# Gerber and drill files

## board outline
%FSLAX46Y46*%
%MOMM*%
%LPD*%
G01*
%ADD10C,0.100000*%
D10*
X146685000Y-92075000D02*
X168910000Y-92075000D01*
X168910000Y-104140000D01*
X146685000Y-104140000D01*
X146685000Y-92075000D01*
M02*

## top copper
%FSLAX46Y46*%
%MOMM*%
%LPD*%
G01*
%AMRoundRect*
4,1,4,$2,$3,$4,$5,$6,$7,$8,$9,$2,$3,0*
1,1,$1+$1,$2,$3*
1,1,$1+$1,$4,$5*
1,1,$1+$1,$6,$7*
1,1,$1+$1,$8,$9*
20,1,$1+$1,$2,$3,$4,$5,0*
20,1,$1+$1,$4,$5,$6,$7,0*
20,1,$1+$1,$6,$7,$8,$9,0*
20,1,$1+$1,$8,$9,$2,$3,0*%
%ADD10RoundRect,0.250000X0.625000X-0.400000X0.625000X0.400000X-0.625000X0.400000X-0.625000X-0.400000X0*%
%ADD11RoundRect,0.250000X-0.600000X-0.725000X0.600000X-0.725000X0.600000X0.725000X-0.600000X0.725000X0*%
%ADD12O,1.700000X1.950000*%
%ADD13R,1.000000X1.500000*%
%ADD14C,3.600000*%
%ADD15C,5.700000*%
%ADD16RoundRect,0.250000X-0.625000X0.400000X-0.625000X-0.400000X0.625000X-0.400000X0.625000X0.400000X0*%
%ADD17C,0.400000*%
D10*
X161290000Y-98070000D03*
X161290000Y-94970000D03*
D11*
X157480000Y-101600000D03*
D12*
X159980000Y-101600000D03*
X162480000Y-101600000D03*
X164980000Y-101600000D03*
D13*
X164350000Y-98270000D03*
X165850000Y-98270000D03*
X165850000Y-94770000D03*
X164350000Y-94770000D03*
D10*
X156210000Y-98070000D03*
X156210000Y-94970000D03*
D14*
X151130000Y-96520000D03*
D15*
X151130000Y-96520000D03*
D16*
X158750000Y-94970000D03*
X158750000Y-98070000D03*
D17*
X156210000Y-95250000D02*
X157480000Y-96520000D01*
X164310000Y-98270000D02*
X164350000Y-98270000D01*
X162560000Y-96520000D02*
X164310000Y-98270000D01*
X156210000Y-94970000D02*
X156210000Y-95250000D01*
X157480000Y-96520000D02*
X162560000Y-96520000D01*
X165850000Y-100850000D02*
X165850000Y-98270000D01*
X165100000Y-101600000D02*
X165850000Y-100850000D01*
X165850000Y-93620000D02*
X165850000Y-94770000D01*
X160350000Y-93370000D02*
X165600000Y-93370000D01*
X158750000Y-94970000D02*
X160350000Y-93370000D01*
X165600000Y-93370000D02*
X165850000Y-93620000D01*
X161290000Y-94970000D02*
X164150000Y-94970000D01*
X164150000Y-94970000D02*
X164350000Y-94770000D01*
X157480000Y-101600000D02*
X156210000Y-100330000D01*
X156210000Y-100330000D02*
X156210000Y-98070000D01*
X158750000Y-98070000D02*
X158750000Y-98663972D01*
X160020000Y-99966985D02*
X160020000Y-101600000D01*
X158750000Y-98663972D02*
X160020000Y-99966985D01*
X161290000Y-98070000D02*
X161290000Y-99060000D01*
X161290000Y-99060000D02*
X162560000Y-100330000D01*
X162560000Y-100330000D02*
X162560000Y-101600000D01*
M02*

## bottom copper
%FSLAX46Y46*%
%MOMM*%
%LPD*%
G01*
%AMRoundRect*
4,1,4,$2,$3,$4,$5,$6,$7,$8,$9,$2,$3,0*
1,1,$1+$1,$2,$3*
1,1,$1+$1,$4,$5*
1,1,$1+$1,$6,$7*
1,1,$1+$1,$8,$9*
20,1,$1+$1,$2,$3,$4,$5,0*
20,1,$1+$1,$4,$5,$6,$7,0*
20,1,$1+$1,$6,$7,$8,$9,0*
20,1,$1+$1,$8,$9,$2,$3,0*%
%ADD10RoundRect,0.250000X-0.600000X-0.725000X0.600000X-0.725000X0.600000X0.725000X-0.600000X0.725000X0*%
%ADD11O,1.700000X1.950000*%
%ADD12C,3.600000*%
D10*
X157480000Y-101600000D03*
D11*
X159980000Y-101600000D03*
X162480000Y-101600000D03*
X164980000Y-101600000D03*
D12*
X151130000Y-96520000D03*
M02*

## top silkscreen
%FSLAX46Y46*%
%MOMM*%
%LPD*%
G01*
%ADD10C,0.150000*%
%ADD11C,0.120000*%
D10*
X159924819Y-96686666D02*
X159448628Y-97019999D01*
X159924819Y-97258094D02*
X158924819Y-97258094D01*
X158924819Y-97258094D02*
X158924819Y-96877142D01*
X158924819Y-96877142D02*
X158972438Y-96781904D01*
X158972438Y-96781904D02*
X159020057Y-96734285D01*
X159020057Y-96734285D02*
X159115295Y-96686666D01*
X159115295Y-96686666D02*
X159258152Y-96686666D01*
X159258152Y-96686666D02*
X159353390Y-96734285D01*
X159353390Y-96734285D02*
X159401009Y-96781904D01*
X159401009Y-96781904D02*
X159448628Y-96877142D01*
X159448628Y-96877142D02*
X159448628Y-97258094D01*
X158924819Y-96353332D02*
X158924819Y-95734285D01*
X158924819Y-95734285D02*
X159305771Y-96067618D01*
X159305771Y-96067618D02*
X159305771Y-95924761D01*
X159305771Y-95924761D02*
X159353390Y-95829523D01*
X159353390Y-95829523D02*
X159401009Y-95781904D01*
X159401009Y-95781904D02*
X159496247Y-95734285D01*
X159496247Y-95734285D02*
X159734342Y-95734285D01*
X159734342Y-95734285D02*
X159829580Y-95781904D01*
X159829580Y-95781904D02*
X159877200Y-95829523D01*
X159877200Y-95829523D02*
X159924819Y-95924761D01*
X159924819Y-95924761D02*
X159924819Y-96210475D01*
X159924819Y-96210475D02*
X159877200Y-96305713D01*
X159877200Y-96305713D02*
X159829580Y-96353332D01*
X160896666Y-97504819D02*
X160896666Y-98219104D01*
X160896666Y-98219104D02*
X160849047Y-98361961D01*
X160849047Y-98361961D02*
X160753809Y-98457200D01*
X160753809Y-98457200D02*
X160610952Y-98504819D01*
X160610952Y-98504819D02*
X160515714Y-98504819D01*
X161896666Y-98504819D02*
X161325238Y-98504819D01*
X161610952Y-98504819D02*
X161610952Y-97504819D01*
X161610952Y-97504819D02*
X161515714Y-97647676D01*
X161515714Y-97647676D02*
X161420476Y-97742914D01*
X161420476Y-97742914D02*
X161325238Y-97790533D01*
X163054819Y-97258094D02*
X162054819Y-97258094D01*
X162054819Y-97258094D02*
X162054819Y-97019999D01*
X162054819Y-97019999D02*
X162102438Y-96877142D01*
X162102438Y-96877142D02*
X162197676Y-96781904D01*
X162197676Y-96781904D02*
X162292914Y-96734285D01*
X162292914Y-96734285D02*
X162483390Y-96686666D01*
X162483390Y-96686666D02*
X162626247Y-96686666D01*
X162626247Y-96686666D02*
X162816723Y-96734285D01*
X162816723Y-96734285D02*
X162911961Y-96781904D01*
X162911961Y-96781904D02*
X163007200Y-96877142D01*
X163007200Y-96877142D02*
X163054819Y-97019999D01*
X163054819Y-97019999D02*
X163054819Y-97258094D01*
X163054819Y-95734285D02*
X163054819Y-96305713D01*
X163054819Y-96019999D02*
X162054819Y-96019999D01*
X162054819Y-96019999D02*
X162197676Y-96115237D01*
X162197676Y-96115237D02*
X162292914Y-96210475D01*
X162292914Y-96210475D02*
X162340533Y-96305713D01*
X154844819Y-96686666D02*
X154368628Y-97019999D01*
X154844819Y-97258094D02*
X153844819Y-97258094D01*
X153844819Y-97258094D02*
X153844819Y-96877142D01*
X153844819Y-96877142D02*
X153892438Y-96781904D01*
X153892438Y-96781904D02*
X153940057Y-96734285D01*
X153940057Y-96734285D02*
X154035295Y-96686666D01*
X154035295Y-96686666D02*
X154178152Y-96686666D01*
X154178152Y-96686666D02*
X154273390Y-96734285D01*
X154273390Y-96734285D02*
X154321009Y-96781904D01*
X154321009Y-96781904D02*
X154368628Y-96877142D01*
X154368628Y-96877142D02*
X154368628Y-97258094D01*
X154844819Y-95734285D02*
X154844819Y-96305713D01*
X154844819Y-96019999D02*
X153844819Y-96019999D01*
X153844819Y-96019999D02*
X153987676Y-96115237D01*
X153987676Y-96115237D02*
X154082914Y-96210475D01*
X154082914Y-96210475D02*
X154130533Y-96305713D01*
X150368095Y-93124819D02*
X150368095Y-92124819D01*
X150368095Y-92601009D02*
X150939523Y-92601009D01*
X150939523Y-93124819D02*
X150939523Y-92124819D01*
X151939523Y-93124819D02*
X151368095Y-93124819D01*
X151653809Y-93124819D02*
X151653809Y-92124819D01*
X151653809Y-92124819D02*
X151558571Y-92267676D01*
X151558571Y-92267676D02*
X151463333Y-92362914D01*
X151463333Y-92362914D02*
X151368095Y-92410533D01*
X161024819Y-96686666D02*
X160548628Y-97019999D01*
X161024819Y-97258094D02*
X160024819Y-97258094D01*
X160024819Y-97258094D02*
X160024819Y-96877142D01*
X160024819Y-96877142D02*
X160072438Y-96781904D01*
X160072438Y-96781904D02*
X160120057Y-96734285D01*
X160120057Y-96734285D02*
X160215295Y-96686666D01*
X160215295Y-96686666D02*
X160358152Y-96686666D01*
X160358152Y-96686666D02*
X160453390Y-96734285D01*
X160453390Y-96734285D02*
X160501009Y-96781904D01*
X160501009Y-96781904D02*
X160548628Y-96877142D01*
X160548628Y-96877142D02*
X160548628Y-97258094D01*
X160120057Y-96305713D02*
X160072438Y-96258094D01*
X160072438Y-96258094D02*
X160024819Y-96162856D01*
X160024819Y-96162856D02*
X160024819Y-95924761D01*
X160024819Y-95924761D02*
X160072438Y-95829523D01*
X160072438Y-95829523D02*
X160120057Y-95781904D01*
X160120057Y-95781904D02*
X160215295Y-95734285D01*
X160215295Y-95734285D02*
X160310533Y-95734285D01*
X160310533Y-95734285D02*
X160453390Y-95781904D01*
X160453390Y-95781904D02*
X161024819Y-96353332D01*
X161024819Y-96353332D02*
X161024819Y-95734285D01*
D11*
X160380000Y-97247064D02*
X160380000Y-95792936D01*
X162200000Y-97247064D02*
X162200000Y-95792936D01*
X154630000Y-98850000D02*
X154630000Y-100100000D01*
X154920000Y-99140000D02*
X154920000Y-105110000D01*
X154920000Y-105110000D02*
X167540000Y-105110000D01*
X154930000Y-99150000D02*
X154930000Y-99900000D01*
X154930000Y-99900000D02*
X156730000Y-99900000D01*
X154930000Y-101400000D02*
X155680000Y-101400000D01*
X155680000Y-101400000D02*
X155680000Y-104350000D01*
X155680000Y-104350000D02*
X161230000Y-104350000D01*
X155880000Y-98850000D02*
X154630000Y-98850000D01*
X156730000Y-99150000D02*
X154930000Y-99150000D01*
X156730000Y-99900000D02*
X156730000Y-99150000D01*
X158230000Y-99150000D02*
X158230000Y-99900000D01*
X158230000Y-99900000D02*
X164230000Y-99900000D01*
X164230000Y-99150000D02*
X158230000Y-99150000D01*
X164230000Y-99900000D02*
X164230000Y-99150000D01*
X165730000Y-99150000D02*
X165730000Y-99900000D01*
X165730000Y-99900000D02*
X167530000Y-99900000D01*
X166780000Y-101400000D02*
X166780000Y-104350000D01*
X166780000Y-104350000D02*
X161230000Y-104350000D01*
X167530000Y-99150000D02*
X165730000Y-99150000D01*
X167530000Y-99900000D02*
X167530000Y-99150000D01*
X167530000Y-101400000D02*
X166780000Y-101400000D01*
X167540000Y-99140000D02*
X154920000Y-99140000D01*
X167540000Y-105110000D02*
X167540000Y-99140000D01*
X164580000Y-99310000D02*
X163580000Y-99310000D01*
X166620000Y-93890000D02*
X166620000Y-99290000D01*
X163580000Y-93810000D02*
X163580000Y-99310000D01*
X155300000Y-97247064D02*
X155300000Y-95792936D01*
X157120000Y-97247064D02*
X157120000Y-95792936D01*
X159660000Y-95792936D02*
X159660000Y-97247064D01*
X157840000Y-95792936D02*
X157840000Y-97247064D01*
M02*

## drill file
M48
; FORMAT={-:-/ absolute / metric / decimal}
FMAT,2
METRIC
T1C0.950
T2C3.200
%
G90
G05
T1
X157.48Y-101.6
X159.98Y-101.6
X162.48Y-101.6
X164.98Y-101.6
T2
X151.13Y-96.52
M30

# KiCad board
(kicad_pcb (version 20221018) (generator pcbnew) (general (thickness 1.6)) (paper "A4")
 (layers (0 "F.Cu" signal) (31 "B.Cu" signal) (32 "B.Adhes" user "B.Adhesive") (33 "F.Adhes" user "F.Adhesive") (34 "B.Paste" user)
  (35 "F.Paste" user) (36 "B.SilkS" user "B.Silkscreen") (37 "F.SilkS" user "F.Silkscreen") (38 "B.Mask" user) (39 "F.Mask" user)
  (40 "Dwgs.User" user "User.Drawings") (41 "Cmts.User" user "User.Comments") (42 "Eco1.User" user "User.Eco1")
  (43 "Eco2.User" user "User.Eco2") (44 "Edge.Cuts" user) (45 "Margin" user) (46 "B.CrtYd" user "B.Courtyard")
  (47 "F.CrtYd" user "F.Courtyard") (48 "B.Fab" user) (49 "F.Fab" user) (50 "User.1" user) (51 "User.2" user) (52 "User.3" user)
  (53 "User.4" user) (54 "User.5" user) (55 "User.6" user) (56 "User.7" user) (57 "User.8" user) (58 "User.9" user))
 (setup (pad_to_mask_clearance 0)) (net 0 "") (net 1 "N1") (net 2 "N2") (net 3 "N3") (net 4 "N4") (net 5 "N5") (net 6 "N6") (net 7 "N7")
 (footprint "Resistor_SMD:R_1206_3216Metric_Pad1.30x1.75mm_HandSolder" (layer "F.Cu") (at 161.29 96.52 90)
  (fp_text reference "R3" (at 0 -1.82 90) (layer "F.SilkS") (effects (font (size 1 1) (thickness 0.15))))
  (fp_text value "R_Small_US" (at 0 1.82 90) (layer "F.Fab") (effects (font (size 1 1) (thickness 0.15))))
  (fp_line (start -0.727064 -0.91) (end 0.727064 -0.91) (stroke (width 0.12) (type solid)) (layer "F.SilkS"))
  (fp_line (start -0.727064 0.91) (end 0.727064 0.91) (stroke (width 0.12) (type solid)) (layer "F.SilkS"))
  (pad "1" smd roundrect (at -1.55 0 90) (size 1.3 1.75) (layers "F.Cu" "F.Paste" "F.Mask") (roundrect_rratio 0.1923076923) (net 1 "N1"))
  (pad "2" smd roundrect (at 1.55 0 90) (size 1.3 1.75) (layers "F.Cu" "F.Paste" "F.Mask") (roundrect_rratio 0.1923076923) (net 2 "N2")))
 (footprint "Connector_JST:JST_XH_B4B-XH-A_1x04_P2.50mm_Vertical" (layer "F.Cu") (at 157.48 101.6)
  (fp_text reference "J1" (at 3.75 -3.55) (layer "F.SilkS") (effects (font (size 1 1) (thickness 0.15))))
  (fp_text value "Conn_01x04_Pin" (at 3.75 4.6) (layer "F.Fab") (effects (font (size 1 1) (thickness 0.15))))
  (fp_line (start -2.85 -2.75) (end -2.85 -1.5) (stroke (width 0.12) (type solid)) (layer "F.SilkS"))
  (fp_line (start -2.56 -2.46) (end -2.56 3.51) (stroke (width 0.12) (type solid)) (layer "F.SilkS"))
  (fp_line (start -2.56 3.51) (end 10.06 3.51) (stroke (width 0.12) (type solid)) (layer "F.SilkS"))
  (fp_line (start -2.55 -2.45) (end -2.55 -1.7) (stroke (width 0.12) (type solid)) (layer "F.SilkS"))
  (fp_line (start -2.55 -1.7) (end -0.75 -1.7) (stroke (width 0.12) (type solid)) (layer "F.SilkS"))
  (fp_line (start -2.55 -0.2) (end -1.8 -0.2) (stroke (width 0.12) (type solid)) (layer "F.SilkS"))
  (fp_line (start -1.8 -0.2) (end -1.8 2.75) (stroke (width 0.12) (type solid)) (layer "F.SilkS"))
  (fp_line (start -1.8 2.75) (end 3.75 2.75) (stroke (width 0.12) (type solid)) (layer "F.SilkS"))
  (fp_line (start -1.6 -2.75) (end -2.85 -2.75) (stroke (width 0.12) (type solid)) (layer "F.SilkS"))
  (fp_line (start -0.75 -2.45) (end -2.55 -2.45) (stroke (width 0.12) (type solid)) (layer "F.SilkS"))
  (fp_line (start -0.75 -1.7) (end -0.75 -2.45) (stroke (width 0.12) (type solid)) (layer "F.SilkS"))
  (fp_line (start 0.75 -2.45) (end 0.75 -1.7) (stroke (width 0.12) (type solid)) (layer "F.SilkS"))
  (fp_line (start 0.75 -1.7) (end 6.75 -1.7) (stroke (width 0.12) (type solid)) (layer "F.SilkS"))
  (fp_line (start 6.75 -2.45) (end 0.75 -2.45) (stroke (width 0.12) (type solid)) (layer "F.SilkS"))
  (fp_line (start 6.75 -1.7) (end 6.75 -2.45) (stroke (width 0.12) (type solid)) (layer "F.SilkS"))
  (fp_line (start 8.25 -2.45) (end 8.25 -1.7) (stroke (width 0.12) (type solid)) (layer "F.SilkS"))
  (fp_line (start 8.25 -1.7) (end 10.05 -1.7) (stroke (width 0.12) (type solid)) (layer "F.SilkS"))
  (fp_line (start 9.3 -0.2) (end 9.3 2.75) (stroke (width 0.12) (type solid)) (layer "F.SilkS"))
  (fp_line (start 9.3 2.75) (end 3.75 2.75) (stroke (width 0.12) (type solid)) (layer "F.SilkS"))
  (fp_line (start 10.05 -2.45) (end 8.25 -2.45) (stroke (width 0.12) (type solid)) (layer "F.SilkS"))
  (fp_line (start 10.05 -1.7) (end 10.05 -2.45) (stroke (width 0.12) (type solid)) (layer "F.SilkS"))
  (fp_line (start 10.05 -0.2) (end 9.3 -0.2) (stroke (width 0.12) (type solid)) (layer "F.SilkS"))
  (fp_line (start 10.06 -2.46) (end -2.56 -2.46) (stroke (width 0.12) (type solid)) (layer "F.SilkS"))
  (fp_line (start 10.06 3.51) (end 10.06 -2.46) (stroke (width 0.12) (type solid)) (layer "F.SilkS"))
  (pad "1" thru_hole roundrect (at 0 0) (size 1.7 1.95) (drill 0.95) (layers "*.Cu" "*.Mask") (roundrect_rratio 0.147059) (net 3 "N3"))
  (pad "2" thru_hole oval (at 2.5 0) (size 1.7 1.95) (drill 0.95) (layers "*.Cu" "*.Mask") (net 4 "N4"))
  (pad "3" thru_hole oval (at 5 0) (size 1.7 1.95) (drill 0.95) (layers "*.Cu" "*.Mask") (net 1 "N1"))
  (pad "4" thru_hole oval (at 7.5 0) (size 1.7 1.95) (drill 0.95) (layers "*.Cu" "*.Mask") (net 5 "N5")))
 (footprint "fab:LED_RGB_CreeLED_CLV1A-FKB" (layer "F.Cu") (at 165.1 96.52 90)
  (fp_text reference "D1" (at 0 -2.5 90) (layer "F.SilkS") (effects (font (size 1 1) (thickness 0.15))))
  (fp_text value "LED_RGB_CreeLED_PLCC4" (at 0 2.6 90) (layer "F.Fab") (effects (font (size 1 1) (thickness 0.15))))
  (fp_line (start -2.79 -0.52) (end -2.79 -1.52) (stroke (width 0.12) (type solid)) (layer "F.SilkS"))
  (fp_line (start 2.63 1.52) (end -2.77 1.52) (stroke (width 0.12) (type solid)) (layer "F.SilkS"))
  (fp_line (start 2.71 -1.52) (end -2.79 -1.52) (stroke (width 0.12) (type solid)) (layer "F.SilkS"))
  (pad "1" smd rect (at -1.75 -0.75 270) (size 1.5 1) (layers "F.Cu" "F.Paste" "F.Mask") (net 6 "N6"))
  (pad "2" smd rect (at -1.75 0.75 270) (size 1.5 1) (layers "F.Cu" "F.Paste" "F.Mask") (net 5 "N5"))
  (pad "3" smd rect (at 1.75 0.75 270) (size 1.5 1) (layers "F.Cu" "F.Paste" "F.Mask") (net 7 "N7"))
  (pad "4" smd rect (at 1.75 -0.75 270) (size 1.5 1) (layers "F.Cu" "F.Paste" "F.Mask") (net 2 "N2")))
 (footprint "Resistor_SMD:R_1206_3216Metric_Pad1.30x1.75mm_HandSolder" (layer "F.Cu") (at 156.21 96.52 90)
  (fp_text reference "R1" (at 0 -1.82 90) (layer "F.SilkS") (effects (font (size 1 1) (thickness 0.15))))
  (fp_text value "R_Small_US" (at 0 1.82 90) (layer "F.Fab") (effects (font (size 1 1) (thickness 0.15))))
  (fp_line (start -0.727064 -0.91) (end 0.727064 -0.91) (stroke (width 0.12) (type solid)) (layer "F.SilkS"))
  (fp_line (start -0.727064 0.91) (end 0.727064 0.91) (stroke (width 0.12) (type solid)) (layer "F.SilkS"))
  (pad "1" smd roundrect (at -1.55 0 90) (size 1.3 1.75) (layers "F.Cu" "F.Paste" "F.Mask") (roundrect_rratio 0.1923076923) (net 3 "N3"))
  (pad "2" smd roundrect (at 1.55 0 90) (size 1.3 1.75) (layers "F.Cu" "F.Paste" "F.Mask") (roundrect_rratio 0.1923076923) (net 6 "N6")))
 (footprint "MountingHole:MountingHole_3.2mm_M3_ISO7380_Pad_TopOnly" (layer "F.Cu") (at 151.13 96.52)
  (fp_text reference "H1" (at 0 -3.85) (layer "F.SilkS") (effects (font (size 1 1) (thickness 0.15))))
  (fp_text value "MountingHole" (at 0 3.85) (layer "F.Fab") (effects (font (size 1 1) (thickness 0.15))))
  (pad "1" thru_hole circle (at 0 0) (size 3.6 3.6) (drill 3.2) (layers "*.Cu" "*.Mask"))
  (pad "1" connect circle (at 0 0) (size 5.7 5.7) (layers "F.Cu" "F.Mask")))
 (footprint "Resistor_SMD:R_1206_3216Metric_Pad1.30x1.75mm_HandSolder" (layer "F.Cu") (at 158.75 96.52 -90)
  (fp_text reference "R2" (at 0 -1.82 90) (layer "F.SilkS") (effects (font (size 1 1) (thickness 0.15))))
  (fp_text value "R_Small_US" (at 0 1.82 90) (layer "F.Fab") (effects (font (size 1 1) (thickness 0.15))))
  (fp_line (start -0.727064 -0.91) (end 0.727064 -0.91) (stroke (width 0.12) (type solid)) (layer "F.SilkS"))
  (fp_line (start -0.727064 0.91) (end 0.727064 0.91) (stroke (width 0.12) (type solid)) (layer "F.SilkS"))
  (pad "1" smd roundrect (at -1.55 0 270) (size 1.3 1.75) (layers "F.Cu" "F.Paste" "F.Mask") (roundrect_rratio 0.1923076923) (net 7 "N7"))
  (pad "2" smd roundrect (at 1.55 0 270) (size 1.3 1.75) (layers "F.Cu" "F.Paste" "F.Mask") (roundrect_rratio 0.1923076923) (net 4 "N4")))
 (gr_rect (start 146.685 92.075) (end 168.91 104.14) (stroke (width 0.1) (type default)) (fill none) (layer "Edge.Cuts"))
 (segment (start 156.21 95.25) (end 157.48 96.52) (width 0.4) (layer "F.Cu") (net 6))
 (segment (start 164.31 98.27) (end 164.35 98.27) (width 0.4) (layer "F.Cu") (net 6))
 (segment (start 162.56 96.52) (end 164.31 98.27) (width 0.4) (layer "F.Cu") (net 6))
 (segment (start 156.21 94.97) (end 156.21 95.25) (width 0.4) (layer "F.Cu") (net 6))
 (segment (start 157.48 96.52) (end 162.56 96.52) (width 0.4) (layer "F.Cu") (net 6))
 (segment (start 165.85 100.85) (end 165.85 98.27) (width 0.4) (layer "F.Cu") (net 5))
 (segment (start 165.1 101.6) (end 165.85 100.85) (width 0.4) (layer "F.Cu") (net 5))
 (segment (start 165.85 93.62) (end 165.85 94.77) (width 0.4) (layer "F.Cu") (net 7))
 (segment (start 160.35 93.37) (end 165.6 93.37) (width 0.4) (layer "F.Cu") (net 7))
 (segment (start 158.75 94.97) (end 160.35 93.37) (width 0.4) (layer "F.Cu") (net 7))
 (segment (start 165.6 93.37) (end 165.85 93.62) (width 0.4) (layer "F.Cu") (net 7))
 (segment (start 161.29 94.97) (end 164.15 94.97) (width 0.4) (layer "F.Cu") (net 2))
 (segment (start 164.15 94.97) (end 164.35 94.77) (width 0.4) (layer "F.Cu") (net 2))
 (segment (start 157.48 101.6) (end 156.21 100.33) (width 0.4) (layer "F.Cu") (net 3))
 (segment (start 156.21 100.33) (end 156.21 98.07) (width 0.4) (layer "F.Cu") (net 3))
 (segment (start 158.75 98.07) (end 158.75 98.663972) (width 0.4) (layer "F.Cu") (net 4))
 (segment (start 160.02 99.966985) (end 160.02 101.6) (width 0.4) (layer "F.Cu") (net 4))
 (segment (start 158.75 98.663972) (end 160.02 99.966985) (width 0.4) (layer "F.Cu") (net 4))
 (segment (start 161.29 98.07) (end 161.29 99.06) (width 0.4) (layer "F.Cu") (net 1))
 (segment (start 161.29 99.06) (end 162.56 100.33) (width 0.4) (layer "F.Cu") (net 1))
 (segment (start 162.56 100.33) (end 162.56 101.6) (width 0.4) (layer "F.Cu") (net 1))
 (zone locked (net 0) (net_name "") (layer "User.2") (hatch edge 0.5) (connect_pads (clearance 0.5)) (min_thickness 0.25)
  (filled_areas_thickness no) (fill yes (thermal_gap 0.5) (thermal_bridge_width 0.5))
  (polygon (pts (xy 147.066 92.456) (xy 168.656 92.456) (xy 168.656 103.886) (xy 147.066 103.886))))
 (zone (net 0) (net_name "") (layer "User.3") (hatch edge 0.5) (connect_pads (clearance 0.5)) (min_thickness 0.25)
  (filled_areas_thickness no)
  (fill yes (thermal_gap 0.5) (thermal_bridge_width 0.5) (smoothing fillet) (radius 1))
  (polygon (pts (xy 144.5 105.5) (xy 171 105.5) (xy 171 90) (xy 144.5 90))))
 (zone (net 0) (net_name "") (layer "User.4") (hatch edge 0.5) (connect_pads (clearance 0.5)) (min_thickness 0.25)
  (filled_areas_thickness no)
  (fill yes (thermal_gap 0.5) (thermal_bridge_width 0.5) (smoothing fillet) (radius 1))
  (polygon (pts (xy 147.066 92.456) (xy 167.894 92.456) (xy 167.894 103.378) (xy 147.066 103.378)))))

